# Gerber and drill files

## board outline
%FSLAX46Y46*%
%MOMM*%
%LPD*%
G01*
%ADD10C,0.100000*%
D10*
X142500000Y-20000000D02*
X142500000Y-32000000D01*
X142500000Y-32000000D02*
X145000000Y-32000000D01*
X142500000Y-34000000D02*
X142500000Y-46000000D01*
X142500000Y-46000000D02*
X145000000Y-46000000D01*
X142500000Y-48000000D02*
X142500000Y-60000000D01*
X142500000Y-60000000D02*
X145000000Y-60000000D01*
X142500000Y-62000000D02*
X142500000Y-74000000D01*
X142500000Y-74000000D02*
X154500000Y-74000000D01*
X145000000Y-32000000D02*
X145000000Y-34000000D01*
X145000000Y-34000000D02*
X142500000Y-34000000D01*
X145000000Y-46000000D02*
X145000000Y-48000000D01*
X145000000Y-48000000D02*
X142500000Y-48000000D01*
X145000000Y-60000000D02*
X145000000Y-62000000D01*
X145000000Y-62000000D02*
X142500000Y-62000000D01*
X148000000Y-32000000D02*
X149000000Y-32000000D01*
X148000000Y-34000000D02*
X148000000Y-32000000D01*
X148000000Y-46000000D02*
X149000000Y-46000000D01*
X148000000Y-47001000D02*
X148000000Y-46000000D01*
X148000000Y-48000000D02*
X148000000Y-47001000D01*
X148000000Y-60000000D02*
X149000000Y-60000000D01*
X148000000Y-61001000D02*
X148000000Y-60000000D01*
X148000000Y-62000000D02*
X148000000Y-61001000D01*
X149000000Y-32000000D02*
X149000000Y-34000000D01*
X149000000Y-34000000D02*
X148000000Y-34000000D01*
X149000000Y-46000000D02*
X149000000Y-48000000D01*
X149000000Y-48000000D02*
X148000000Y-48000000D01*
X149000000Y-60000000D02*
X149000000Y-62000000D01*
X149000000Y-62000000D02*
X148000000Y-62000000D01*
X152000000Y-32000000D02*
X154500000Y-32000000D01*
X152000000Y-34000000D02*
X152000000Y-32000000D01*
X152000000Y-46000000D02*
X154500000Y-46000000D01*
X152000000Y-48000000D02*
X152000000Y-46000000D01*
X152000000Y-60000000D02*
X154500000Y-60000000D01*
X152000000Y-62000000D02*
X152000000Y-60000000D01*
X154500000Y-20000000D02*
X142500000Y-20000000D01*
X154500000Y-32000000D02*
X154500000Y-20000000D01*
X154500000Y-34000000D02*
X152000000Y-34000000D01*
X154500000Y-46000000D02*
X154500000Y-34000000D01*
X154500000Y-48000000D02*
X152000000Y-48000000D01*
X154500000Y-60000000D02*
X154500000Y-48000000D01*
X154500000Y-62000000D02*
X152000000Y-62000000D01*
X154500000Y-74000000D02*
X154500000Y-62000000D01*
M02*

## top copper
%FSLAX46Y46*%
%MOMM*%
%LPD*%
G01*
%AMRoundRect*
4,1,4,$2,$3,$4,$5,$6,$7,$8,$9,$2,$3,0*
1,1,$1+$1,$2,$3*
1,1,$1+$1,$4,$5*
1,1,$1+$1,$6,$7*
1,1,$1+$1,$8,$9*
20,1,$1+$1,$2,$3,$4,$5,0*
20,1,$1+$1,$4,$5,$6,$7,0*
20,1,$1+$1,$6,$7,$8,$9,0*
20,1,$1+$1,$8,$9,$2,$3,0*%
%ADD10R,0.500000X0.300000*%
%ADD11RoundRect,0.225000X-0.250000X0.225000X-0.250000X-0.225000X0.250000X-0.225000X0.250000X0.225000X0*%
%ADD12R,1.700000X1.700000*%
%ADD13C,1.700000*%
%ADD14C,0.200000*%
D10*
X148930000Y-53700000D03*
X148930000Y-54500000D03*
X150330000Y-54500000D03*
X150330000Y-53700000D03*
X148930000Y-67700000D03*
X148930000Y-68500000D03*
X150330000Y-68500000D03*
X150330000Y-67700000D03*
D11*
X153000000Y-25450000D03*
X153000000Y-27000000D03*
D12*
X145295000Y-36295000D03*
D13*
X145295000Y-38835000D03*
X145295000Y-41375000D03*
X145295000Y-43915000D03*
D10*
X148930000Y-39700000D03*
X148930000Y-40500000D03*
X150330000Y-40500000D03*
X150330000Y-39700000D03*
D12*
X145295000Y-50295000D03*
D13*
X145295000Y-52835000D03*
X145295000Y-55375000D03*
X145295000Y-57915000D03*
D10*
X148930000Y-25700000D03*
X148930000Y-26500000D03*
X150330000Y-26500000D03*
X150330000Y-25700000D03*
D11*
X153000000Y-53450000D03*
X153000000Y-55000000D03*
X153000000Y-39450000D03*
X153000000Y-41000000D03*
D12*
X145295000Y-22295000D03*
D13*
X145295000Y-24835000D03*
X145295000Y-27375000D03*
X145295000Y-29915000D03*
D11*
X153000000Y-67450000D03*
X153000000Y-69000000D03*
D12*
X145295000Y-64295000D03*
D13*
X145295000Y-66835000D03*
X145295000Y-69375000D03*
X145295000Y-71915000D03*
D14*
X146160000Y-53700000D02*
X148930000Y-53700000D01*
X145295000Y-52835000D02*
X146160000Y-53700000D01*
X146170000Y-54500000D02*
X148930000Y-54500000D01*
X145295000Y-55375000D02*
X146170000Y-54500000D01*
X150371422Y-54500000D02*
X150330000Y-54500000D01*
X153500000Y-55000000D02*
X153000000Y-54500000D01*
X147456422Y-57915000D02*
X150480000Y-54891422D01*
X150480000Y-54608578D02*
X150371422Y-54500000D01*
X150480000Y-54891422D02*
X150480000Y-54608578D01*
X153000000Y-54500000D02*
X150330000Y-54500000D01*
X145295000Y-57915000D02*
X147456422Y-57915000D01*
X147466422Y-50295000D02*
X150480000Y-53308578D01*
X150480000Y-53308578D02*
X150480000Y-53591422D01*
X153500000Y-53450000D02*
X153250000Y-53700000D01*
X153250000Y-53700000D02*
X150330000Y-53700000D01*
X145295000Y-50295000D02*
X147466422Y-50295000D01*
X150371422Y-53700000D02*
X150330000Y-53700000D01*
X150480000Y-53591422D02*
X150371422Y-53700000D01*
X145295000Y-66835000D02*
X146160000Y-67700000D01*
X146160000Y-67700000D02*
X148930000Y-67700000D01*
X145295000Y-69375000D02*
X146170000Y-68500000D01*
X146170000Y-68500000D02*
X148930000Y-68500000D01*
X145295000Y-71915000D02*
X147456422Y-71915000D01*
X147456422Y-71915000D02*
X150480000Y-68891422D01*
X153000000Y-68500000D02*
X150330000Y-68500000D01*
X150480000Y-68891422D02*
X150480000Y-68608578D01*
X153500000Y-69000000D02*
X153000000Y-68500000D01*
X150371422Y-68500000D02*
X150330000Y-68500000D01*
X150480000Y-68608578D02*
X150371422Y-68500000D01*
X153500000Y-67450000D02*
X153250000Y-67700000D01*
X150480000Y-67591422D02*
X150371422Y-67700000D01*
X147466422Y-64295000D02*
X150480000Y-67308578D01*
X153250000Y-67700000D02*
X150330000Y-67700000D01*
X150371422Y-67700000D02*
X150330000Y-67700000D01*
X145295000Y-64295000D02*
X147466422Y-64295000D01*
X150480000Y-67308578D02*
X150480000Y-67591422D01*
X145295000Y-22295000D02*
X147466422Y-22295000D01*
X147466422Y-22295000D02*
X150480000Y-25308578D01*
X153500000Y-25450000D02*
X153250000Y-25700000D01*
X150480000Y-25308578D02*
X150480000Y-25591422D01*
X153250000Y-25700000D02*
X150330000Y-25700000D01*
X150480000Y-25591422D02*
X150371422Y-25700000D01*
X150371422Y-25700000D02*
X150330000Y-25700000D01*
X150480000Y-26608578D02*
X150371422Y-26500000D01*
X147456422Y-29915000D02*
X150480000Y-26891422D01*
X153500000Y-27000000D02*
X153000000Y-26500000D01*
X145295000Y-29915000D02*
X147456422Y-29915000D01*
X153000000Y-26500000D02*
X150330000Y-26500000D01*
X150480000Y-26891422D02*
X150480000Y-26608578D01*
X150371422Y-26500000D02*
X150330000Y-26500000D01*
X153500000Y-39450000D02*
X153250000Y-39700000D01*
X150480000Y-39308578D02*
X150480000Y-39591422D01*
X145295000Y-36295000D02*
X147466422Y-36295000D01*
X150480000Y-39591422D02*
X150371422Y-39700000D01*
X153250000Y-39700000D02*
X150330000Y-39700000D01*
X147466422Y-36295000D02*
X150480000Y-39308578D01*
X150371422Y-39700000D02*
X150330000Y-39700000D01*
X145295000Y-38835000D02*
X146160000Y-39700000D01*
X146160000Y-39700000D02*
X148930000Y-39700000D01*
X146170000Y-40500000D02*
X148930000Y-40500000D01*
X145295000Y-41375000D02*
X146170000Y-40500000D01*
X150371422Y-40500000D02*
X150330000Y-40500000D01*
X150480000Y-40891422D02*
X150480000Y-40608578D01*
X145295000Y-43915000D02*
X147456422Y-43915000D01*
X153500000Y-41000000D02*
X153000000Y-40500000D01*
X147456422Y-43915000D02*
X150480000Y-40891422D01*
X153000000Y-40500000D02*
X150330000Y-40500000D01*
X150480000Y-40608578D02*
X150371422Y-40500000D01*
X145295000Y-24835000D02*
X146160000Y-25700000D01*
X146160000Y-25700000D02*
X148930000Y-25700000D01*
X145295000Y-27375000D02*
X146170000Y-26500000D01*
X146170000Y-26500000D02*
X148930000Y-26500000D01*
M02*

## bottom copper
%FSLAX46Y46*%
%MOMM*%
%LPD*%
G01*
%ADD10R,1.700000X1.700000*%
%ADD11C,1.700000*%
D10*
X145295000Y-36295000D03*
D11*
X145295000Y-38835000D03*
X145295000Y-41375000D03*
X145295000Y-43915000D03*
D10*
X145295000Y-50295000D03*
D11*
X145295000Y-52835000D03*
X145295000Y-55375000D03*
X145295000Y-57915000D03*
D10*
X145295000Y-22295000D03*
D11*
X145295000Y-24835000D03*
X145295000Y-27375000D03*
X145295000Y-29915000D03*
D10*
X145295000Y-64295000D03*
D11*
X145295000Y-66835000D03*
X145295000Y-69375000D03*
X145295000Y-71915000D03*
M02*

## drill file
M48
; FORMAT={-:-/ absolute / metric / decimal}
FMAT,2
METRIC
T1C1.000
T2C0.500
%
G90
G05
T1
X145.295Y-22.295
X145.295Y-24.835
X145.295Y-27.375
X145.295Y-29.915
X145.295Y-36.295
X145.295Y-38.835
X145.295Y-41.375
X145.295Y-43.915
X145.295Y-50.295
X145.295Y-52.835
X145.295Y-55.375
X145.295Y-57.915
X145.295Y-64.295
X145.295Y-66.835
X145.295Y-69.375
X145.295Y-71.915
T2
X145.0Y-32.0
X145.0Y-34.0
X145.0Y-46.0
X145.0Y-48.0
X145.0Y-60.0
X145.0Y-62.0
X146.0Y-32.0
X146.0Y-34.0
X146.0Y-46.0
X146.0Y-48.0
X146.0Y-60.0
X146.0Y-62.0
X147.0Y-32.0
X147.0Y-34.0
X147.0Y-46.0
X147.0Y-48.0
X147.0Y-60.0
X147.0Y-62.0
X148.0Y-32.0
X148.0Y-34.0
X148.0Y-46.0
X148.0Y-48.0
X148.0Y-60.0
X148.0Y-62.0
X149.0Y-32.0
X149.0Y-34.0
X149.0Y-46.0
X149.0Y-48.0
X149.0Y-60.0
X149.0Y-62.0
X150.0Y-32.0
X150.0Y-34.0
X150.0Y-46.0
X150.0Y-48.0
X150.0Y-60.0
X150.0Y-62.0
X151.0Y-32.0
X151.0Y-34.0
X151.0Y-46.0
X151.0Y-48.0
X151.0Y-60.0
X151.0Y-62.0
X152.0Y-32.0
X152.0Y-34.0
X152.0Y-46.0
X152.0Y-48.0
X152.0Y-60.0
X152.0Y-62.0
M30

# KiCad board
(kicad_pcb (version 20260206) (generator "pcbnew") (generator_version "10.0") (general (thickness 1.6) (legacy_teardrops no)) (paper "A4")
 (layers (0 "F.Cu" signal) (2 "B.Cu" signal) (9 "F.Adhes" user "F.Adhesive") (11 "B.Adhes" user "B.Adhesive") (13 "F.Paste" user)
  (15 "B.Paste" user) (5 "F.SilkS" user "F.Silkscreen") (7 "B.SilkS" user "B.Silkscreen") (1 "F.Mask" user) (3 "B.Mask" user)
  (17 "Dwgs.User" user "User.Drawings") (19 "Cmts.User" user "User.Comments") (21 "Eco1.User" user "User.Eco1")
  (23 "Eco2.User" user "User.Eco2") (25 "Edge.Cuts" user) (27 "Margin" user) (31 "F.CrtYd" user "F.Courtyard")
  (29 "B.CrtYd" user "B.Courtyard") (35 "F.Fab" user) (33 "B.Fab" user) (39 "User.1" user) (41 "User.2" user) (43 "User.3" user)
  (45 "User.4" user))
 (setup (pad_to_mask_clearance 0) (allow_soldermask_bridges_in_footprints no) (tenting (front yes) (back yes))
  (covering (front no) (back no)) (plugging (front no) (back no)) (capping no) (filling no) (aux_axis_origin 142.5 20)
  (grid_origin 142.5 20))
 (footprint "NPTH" (layer "F.Cu") (at 150 48)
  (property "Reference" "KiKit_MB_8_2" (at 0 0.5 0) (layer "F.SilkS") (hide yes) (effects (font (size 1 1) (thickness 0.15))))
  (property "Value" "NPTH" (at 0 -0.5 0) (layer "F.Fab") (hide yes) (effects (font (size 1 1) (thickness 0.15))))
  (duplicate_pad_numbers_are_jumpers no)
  (pad "" np_thru_hole circle (at 0 0) (size 0.5 0.5) (drill 0.5) (layers "*.Cu" "*.Mask")))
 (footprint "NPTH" (layer "F.Cu") (at 152 34)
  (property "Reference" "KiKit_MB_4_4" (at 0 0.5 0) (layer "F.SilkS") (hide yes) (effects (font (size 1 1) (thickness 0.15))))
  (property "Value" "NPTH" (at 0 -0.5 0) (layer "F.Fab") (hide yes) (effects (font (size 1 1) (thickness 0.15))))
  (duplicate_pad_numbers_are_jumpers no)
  (pad "" np_thru_hole circle (at 0 0) (size 0.5 0.5) (drill 0.5) (layers "*.Cu" "*.Mask")))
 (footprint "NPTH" (layer "F.Cu") (at 149 62)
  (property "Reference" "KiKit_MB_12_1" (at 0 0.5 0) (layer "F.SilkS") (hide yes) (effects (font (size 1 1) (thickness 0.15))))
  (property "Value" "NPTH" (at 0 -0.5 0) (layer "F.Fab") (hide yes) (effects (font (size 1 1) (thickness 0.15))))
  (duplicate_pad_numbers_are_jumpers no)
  (pad "" np_thru_hole circle (at 0 0) (size 0.5 0.5) (drill 0.5) (layers "*.Cu" "*.Mask")))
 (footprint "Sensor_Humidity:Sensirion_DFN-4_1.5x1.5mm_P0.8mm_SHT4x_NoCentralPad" (layer "F.Cu") (at 149.63 54.1)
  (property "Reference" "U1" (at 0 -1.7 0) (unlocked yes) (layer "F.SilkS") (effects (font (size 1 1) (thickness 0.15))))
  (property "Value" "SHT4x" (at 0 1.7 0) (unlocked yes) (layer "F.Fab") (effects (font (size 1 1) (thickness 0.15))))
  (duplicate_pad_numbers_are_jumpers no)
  (pad "1" smd rect (at -0.7 -0.4) (size 0.5 0.3) (layers "F.Cu" "F.Mask" "F.Paste") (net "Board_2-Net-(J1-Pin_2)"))
  (pad "2" smd rect (at -0.7 0.4) (size 0.5 0.3) (layers "F.Cu" "F.Mask" "F.Paste") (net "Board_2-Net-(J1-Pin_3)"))
  (pad "3" smd rect (at 0.7 0.4) (size 0.5 0.3) (layers "F.Cu" "F.Mask" "F.Paste") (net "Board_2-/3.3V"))
  (pad "4" smd rect (at 0.7 -0.4) (size 0.5 0.3) (layers "F.Cu" "F.Mask" "F.Paste") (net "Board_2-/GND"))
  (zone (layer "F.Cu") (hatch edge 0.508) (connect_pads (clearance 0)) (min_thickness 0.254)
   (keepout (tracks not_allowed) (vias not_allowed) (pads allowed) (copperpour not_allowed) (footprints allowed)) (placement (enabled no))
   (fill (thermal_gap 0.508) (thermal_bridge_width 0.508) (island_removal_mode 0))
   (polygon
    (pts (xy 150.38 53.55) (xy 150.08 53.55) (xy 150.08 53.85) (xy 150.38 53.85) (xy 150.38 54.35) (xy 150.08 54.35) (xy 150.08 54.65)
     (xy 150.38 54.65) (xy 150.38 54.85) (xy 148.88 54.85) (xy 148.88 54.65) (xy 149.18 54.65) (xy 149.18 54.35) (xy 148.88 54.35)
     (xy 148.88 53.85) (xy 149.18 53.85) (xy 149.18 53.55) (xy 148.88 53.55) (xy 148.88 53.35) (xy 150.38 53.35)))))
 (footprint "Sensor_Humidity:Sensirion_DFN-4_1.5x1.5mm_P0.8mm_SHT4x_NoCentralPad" (layer "F.Cu") (at 149.63 68.1)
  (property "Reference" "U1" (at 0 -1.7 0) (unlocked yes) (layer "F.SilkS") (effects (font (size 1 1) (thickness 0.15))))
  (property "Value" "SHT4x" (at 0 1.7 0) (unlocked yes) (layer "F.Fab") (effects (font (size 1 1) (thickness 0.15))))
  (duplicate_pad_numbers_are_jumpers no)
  (pad "1" smd rect (at -0.7 -0.4) (size 0.5 0.3) (layers "F.Cu" "F.Mask" "F.Paste") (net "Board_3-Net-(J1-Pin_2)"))
  (pad "2" smd rect (at -0.7 0.4) (size 0.5 0.3) (layers "F.Cu" "F.Mask" "F.Paste") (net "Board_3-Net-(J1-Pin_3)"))
  (pad "3" smd rect (at 0.7 0.4) (size 0.5 0.3) (layers "F.Cu" "F.Mask" "F.Paste") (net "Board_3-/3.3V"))
  (pad "4" smd rect (at 0.7 -0.4) (size 0.5 0.3) (layers "F.Cu" "F.Mask" "F.Paste") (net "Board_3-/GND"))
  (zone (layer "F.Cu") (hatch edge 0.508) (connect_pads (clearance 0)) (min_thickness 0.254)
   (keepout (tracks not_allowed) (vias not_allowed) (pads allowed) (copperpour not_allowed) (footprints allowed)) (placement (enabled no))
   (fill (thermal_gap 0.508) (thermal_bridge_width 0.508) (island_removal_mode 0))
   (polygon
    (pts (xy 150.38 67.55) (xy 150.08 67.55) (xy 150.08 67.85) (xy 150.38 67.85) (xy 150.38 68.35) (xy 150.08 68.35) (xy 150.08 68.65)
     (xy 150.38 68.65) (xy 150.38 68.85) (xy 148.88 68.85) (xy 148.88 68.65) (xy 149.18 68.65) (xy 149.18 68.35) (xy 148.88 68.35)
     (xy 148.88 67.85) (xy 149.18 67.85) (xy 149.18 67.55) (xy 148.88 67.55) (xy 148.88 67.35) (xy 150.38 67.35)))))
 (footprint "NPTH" (layer "F.Cu") (at 147 48)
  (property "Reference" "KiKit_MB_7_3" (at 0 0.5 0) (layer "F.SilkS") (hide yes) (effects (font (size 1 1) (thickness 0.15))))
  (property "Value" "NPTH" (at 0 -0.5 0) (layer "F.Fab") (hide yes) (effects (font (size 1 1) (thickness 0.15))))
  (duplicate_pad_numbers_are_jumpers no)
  (pad "" np_thru_hole circle (at 0 0) (size 0.5 0.5) (drill 0.5) (layers "*.Cu" "*.Mask")))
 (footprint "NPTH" (layer "F.Cu") (at 146 46)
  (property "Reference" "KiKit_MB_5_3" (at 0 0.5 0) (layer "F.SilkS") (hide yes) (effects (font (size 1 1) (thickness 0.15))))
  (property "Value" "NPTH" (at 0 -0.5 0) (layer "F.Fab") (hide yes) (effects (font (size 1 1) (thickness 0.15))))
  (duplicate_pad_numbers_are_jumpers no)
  (pad "" np_thru_hole circle (at 0 0) (size 0.5 0.5) (drill 0.5) (layers "*.Cu" "*.Mask")))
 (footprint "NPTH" (layer "F.Cu") (at 145 34)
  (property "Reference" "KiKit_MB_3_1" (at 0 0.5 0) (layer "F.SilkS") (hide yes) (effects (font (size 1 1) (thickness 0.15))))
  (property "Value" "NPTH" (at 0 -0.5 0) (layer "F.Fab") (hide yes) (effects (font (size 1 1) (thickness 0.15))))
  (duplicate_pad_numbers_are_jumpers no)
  (pad "" np_thru_hole circle (at 0 0) (size 0.5 0.5) (drill 0.5) (layers "*.Cu" "*.Mask")))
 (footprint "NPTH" (layer "F.Cu") (at 145 62)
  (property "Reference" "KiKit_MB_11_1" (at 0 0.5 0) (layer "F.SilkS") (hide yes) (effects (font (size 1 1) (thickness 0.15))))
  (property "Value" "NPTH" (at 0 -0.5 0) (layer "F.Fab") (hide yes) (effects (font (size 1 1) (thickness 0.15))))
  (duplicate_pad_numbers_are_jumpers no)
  (pad "" np_thru_hole circle (at 0 0) (size 0.5 0.5) (drill 0.5) (layers "*.Cu" "*.Mask")))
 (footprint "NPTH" (layer "F.Cu") (at 151 62)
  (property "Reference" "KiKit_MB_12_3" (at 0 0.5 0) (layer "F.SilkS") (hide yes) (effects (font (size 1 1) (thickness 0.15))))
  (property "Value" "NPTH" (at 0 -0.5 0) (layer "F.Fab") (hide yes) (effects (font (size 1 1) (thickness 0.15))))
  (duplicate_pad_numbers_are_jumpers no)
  (pad "" np_thru_hole circle (at 0 0) (size 0.5 0.5) (drill 0.5) (layers "*.Cu" "*.Mask")))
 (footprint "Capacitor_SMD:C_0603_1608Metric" (layer "F.Cu") (at 153 26.225 -90)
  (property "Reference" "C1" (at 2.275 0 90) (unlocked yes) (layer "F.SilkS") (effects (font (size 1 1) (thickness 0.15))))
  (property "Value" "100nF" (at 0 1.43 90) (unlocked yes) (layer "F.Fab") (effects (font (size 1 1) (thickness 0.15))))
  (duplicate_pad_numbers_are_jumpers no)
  (pad "1" smd roundrect (at -0.775 0 270) (size 0.9 0.95) (layers "F.Cu" "F.Mask" "F.Paste") (roundrect_rratio 0.25) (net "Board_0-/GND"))
  (pad "2" smd roundrect (at 0.775 0 270) (size 0.9 0.95) (layers "F.Cu" "F.Mask" "F.Paste") (roundrect_rratio 0.25) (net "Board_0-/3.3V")))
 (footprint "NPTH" (layer "F.Cu") (at 149 48)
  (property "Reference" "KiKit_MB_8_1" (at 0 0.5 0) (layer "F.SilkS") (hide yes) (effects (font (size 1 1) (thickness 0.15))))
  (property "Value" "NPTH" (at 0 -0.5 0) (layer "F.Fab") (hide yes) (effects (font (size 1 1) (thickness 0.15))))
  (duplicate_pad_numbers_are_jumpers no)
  (pad "" np_thru_hole circle (at 0 0) (size 0.5 0.5) (drill 0.5) (layers "*.Cu" "*.Mask")))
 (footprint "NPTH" (layer "F.Cu") (at 148 32)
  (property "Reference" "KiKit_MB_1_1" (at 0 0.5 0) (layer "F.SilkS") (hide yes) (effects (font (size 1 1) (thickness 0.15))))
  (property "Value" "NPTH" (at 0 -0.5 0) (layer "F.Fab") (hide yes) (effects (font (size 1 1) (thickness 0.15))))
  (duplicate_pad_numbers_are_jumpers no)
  (pad "" np_thru_hole circle (at 0 0) (size 0.5 0.5) (drill 0.5) (layers "*.Cu" "*.Mask")))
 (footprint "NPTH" (layer "F.Cu") (at 145 32)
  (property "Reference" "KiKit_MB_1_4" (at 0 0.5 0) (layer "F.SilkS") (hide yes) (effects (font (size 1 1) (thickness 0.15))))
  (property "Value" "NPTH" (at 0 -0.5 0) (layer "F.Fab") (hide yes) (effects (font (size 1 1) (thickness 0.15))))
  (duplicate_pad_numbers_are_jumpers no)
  (pad "" np_thru_hole circle (at 0 0) (size 0.5 0.5) (drill 0.5) (layers "*.Cu" "*.Mask")))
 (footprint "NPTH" (layer "F.Cu") (at 147 32)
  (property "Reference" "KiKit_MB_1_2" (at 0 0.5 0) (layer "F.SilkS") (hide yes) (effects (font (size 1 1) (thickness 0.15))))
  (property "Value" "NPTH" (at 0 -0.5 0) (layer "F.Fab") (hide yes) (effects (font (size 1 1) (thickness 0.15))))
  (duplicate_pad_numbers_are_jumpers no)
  (pad "" np_thru_hole circle (at 0 0) (size 0.5 0.5) (drill 0.5) (layers "*.Cu" "*.Mask")))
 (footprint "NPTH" (layer "F.Cu") (at 146 48)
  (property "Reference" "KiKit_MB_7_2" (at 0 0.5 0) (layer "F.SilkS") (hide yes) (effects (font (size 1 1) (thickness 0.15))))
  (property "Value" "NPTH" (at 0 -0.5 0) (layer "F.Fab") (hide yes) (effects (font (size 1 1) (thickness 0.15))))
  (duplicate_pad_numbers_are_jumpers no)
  (pad "" np_thru_hole circle (at 0 0) (size 0.5 0.5) (drill 0.5) (layers "*.Cu" "*.Mask")))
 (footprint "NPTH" (layer "F.Cu") (at 146 60)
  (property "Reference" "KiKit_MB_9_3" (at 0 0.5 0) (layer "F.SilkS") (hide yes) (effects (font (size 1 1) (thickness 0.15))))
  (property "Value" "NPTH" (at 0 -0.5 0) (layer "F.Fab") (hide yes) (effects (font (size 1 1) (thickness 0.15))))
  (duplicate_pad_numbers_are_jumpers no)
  (pad "" np_thru_hole circle (at 0 0) (size 0.5 0.5) (drill 0.5) (layers "*.Cu" "*.Mask")))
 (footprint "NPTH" (layer "F.Cu") (at 152 62)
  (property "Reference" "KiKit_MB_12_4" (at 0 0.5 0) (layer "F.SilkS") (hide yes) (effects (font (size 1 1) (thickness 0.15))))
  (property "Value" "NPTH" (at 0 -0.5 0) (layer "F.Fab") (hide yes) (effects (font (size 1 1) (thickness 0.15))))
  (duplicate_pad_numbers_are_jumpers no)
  (pad "" np_thru_hole circle (at 0 0) (size 0.5 0.5) (drill 0.5) (layers "*.Cu" "*.Mask")))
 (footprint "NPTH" (layer "F.Cu") (at 148 60)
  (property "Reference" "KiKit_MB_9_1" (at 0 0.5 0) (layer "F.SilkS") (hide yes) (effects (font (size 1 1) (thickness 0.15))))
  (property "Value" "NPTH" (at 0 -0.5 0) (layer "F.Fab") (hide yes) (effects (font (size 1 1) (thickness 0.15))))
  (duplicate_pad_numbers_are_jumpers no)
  (pad "" np_thru_hole circle (at 0 0) (size 0.5 0.5) (drill 0.5) (layers "*.Cu" "*.Mask")))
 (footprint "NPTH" (layer "F.Cu") (at 150 62)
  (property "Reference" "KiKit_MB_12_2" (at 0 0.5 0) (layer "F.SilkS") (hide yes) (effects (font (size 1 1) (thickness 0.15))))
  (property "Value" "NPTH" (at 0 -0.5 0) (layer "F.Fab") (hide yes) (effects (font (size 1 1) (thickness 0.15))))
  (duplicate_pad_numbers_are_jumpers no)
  (pad "" np_thru_hole circle (at 0 0) (size 0.5 0.5) (drill 0.5) (layers "*.Cu" "*.Mask")))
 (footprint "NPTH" (layer "F.Cu") (at 150 46)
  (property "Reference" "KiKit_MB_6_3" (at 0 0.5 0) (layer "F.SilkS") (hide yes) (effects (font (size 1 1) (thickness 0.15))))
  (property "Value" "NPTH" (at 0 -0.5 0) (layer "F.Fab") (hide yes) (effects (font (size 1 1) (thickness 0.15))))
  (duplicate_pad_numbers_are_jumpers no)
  (pad "" np_thru_hole circle (at 0 0) (size 0.5 0.5) (drill 0.5) (layers "*.Cu" "*.Mask")))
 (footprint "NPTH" (layer "F.Cu") (at 147 60)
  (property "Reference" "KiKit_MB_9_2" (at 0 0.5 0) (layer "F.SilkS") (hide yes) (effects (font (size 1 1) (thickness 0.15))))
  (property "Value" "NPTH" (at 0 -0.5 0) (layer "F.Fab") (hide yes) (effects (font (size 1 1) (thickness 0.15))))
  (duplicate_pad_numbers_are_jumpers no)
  (pad "" np_thru_hole circle (at 0 0) (size 0.5 0.5) (drill 0.5) (layers "*.Cu" "*.Mask")))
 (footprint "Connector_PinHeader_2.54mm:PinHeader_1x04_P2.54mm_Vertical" (layer "F.Cu") (at 145.295 36.295)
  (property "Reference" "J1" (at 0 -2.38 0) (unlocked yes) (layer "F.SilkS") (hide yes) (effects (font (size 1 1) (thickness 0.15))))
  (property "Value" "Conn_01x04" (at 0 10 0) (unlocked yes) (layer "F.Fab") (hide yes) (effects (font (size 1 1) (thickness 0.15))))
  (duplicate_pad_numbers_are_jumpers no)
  (pad "1" thru_hole rect (at 0 0) (size 1.7 1.7) (drill 1) (layers "*.Cu" "*.Mask") (remove_unused_layers no) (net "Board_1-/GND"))
  (pad "2" thru_hole circle (at 0 2.54) (size 1.7 1.7) (drill 1) (layers "*.Cu" "*.Mask") (remove_unused_layers no)
   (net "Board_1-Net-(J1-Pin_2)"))
  (pad "3" thru_hole circle (at 0 5.08) (size 1.7 1.7) (drill 1) (layers "*.Cu" "*.Mask") (remove_unused_layers no)
   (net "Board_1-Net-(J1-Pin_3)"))
  (pad "4" thru_hole circle (at 0 7.62) (size 1.7 1.7) (drill 1) (layers "*.Cu" "*.Mask") (remove_unused_layers no) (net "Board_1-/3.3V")))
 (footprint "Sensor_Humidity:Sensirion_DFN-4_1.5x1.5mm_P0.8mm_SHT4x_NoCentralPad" (layer "F.Cu") (at 149.63 40.1)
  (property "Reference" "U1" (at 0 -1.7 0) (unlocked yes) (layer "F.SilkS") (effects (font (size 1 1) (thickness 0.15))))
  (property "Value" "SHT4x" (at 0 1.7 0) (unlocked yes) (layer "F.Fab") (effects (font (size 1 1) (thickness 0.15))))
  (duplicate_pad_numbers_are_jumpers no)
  (pad "1" smd rect (at -0.7 -0.4) (size 0.5 0.3) (layers "F.Cu" "F.Mask" "F.Paste") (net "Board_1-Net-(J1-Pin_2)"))
  (pad "2" smd rect (at -0.7 0.4) (size 0.5 0.3) (layers "F.Cu" "F.Mask" "F.Paste") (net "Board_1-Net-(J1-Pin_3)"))
  (pad "3" smd rect (at 0.7 0.4) (size 0.5 0.3) (layers "F.Cu" "F.Mask" "F.Paste") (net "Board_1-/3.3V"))
  (pad "4" smd rect (at 0.7 -0.4) (size 0.5 0.3) (layers "F.Cu" "F.Mask" "F.Paste") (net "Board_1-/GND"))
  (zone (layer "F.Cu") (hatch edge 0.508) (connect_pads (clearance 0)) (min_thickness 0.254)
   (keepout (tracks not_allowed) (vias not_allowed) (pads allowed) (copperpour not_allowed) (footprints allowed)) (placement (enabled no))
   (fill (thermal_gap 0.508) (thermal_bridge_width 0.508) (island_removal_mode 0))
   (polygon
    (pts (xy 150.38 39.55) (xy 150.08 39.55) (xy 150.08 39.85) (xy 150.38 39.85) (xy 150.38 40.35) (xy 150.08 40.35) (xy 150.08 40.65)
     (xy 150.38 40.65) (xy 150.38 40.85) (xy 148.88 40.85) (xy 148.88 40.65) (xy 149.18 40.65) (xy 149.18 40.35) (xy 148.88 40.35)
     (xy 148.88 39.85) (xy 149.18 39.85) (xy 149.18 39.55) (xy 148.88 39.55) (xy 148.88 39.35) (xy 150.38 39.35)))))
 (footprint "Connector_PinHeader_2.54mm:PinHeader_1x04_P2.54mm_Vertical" (layer "F.Cu") (at 145.295 50.295)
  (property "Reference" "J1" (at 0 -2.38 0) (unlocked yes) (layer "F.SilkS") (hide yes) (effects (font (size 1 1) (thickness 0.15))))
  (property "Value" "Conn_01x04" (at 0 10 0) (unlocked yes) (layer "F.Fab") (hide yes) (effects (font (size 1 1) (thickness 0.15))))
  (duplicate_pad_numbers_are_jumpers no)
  (pad "1" thru_hole rect (at 0 0) (size 1.7 1.7) (drill 1) (layers "*.Cu" "*.Mask") (remove_unused_layers no) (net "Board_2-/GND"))
  (pad "2" thru_hole circle (at 0 2.54) (size 1.7 1.7) (drill 1) (layers "*.Cu" "*.Mask") (remove_unused_layers no)
   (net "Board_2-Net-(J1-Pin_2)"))
  (pad "3" thru_hole circle (at 0 5.08) (size 1.7 1.7) (drill 1) (layers "*.Cu" "*.Mask") (remove_unused_layers no)
   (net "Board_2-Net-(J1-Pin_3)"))
  (pad "4" thru_hole circle (at 0 7.62) (size 1.7 1.7) (drill 1) (layers "*.Cu" "*.Mask") (remove_unused_layers no) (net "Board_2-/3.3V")))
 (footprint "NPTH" (layer "F.Cu") (at 151 32)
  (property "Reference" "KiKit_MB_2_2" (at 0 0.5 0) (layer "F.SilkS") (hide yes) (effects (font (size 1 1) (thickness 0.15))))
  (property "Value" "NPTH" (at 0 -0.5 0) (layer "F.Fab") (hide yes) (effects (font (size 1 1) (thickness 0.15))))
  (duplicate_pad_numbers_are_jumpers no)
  (pad "" np_thru_hole circle (at 0 0) (size 0.5 0.5) (drill 0.5) (layers "*.Cu" "*.Mask")))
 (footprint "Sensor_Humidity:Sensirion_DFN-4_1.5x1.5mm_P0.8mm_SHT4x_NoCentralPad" (layer "F.Cu") (at 149.63 26.1)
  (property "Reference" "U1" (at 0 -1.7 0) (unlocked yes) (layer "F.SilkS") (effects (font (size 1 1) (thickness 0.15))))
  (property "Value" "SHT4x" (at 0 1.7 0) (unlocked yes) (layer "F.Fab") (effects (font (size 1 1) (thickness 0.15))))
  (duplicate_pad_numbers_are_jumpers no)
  (pad "1" smd rect (at -0.7 -0.4) (size 0.5 0.3) (layers "F.Cu" "F.Mask" "F.Paste") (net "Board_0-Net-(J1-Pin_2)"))
  (pad "2" smd rect (at -0.7 0.4) (size 0.5 0.3) (layers "F.Cu" "F.Mask" "F.Paste") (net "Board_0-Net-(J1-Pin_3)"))
  (pad "3" smd rect (at 0.7 0.4) (size 0.5 0.3) (layers "F.Cu" "F.Mask" "F.Paste") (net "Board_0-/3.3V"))
  (pad "4" smd rect (at 0.7 -0.4) (size 0.5 0.3) (layers "F.Cu" "F.Mask" "F.Paste") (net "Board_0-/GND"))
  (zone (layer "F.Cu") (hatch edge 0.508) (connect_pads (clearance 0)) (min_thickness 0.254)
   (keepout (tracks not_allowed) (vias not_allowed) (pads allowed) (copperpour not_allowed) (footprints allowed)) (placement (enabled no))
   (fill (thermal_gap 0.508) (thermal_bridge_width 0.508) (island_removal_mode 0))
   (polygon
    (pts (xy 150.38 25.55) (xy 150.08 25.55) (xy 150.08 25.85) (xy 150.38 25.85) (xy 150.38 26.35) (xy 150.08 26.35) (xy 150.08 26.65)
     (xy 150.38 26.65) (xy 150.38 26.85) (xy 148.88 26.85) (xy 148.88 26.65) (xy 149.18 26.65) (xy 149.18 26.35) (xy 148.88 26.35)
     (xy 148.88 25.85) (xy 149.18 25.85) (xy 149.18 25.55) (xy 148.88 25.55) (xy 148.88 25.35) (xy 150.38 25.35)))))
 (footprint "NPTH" (layer "F.Cu") (at 152 60)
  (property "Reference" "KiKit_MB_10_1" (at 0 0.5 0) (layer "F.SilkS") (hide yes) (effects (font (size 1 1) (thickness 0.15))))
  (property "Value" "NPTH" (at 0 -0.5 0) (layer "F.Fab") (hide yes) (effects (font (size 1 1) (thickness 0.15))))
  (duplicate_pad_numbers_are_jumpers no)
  (pad "" np_thru_hole circle (at 0 0) (size 0.5 0.5) (drill 0.5) (layers "*.Cu" "*.Mask")))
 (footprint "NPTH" (layer "F.Cu") (at 148 34)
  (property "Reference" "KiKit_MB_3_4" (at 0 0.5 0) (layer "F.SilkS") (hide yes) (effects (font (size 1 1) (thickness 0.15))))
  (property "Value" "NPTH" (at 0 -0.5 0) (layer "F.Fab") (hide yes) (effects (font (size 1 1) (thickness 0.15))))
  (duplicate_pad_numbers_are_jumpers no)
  (pad "" np_thru_hole circle (at 0 0) (size 0.5 0.5) (drill 0.5) (layers "*.Cu" "*.Mask")))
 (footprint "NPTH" (layer "F.Cu") (at 145 48)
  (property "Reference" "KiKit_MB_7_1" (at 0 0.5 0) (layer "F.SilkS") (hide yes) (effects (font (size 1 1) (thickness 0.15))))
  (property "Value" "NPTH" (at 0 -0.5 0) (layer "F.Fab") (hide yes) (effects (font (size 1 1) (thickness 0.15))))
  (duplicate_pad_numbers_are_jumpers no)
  (pad "" np_thru_hole circle (at 0 0) (size 0.5 0.5) (drill 0.5) (layers "*.Cu" "*.Mask")))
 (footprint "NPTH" (layer "F.Cu") (at 149 32)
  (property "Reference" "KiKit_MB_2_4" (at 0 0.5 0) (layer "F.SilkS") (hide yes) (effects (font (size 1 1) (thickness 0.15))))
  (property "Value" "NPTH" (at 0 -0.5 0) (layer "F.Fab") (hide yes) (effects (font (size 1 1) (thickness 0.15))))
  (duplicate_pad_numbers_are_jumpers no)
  (pad "" np_thru_hole circle (at 0 0) (size 0.5 0.5) (drill 0.5) (layers "*.Cu" "*.Mask")))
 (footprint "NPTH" (layer "F.Cu") (at 148 62)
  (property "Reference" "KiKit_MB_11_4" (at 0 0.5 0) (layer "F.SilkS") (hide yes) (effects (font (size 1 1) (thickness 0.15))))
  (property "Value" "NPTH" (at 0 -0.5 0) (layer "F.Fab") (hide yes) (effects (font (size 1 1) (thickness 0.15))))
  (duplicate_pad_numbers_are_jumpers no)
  (pad "" np_thru_hole circle (at 0 0) (size 0.5 0.5) (drill 0.5) (layers "*.Cu" "*.Mask")))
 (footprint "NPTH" (layer "F.Cu") (at 151 48)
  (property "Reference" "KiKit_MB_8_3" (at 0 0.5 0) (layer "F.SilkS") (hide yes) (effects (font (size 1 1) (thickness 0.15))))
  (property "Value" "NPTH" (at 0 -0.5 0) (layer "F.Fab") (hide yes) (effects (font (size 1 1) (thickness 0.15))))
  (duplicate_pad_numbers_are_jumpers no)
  (pad "" np_thru_hole circle (at 0 0) (size 0.5 0.5) (drill 0.5) (layers "*.Cu" "*.Mask")))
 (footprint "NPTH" (layer "F.Cu") (at 148 48)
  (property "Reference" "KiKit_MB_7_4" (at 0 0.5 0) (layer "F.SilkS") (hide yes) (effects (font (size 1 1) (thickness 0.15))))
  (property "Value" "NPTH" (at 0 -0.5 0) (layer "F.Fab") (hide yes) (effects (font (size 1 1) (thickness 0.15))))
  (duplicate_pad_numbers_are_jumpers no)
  (pad "" np_thru_hole circle (at 0 0) (size 0.5 0.5) (drill 0.5) (layers "*.Cu" "*.Mask")))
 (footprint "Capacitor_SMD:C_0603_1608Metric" (layer "F.Cu") (at 153 54.225 -90)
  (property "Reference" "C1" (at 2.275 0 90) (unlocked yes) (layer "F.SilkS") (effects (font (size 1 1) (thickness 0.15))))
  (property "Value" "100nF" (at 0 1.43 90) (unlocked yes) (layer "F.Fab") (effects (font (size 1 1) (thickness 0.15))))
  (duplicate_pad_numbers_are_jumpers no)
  (pad "1" smd roundrect (at -0.775 0 270) (size 0.9 0.95) (layers "F.Cu" "F.Mask" "F.Paste") (roundrect_rratio 0.25) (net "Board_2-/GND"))
  (pad "2" smd roundrect (at 0.775 0 270) (size 0.9 0.95) (layers "F.Cu" "F.Mask" "F.Paste") (roundrect_rratio 0.25) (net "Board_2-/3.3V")))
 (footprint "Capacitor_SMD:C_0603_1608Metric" (layer "F.Cu") (at 153 40.225 -90)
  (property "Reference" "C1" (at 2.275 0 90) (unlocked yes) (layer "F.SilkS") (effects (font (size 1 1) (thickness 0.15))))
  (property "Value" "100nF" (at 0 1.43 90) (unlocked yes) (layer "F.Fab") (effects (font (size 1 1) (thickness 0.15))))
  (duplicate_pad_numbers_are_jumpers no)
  (pad "1" smd roundrect (at -0.775 0 270) (size 0.9 0.95) (layers "F.Cu" "F.Mask" "F.Paste") (roundrect_rratio 0.25) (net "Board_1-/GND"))
  (pad "2" smd roundrect (at 0.775 0 270) (size 0.9 0.95) (layers "F.Cu" "F.Mask" "F.Paste") (roundrect_rratio 0.25) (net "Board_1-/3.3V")))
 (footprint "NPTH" (layer "F.Cu") (at 152 32)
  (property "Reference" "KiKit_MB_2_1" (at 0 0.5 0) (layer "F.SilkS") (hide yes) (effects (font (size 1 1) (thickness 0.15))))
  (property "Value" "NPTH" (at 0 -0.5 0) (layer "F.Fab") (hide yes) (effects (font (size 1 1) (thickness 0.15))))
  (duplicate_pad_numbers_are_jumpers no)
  (pad "" np_thru_hole circle (at 0 0) (size 0.5 0.5) (drill 0.5) (layers "*.Cu" "*.Mask")))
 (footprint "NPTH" (layer "F.Cu") (at 146 62)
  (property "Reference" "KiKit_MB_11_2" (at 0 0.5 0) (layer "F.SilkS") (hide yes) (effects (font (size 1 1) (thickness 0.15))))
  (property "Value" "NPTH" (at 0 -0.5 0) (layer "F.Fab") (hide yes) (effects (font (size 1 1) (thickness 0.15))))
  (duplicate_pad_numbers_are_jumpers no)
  (pad "" np_thru_hole circle (at 0 0) (size 0.5 0.5) (drill 0.5) (layers "*.Cu" "*.Mask")))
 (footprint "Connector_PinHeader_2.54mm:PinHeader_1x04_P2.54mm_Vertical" (layer "F.Cu") (at 145.295 22.295)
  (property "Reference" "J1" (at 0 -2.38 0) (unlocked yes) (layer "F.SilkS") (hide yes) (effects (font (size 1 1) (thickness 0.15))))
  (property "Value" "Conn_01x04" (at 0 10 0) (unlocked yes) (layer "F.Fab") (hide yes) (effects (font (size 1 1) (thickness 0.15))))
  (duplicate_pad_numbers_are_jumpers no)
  (pad "1" thru_hole rect (at 0 0) (size 1.7 1.7) (drill 1) (layers "*.Cu" "*.Mask") (remove_unused_layers no) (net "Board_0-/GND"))
  (pad "2" thru_hole circle (at 0 2.54) (size 1.7 1.7) (drill 1) (layers "*.Cu" "*.Mask") (remove_unused_layers no)
   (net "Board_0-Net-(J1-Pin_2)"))
  (pad "3" thru_hole circle (at 0 5.08) (size 1.7 1.7) (drill 1) (layers "*.Cu" "*.Mask") (remove_unused_layers no)
   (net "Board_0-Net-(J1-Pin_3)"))
  (pad "4" thru_hole circle (at 0 7.62) (size 1.7 1.7) (drill 1) (layers "*.Cu" "*.Mask") (remove_unused_layers no) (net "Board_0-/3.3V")))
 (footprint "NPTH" (layer "F.Cu") (at 146 34)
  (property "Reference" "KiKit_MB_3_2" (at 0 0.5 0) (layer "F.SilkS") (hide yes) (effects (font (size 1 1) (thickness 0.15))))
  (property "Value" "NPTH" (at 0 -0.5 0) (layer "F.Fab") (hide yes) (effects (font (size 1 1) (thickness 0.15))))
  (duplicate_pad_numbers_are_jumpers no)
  (pad "" np_thru_hole circle (at 0 0) (size 0.5 0.5) (drill 0.5) (layers "*.Cu" "*.Mask")))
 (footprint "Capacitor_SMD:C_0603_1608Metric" (layer "F.Cu") (at 153 68.225 -90)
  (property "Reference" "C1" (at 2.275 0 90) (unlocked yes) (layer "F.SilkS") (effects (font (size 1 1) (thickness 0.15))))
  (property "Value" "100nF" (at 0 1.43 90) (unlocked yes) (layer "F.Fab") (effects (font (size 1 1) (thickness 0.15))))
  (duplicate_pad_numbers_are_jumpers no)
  (pad "1" smd roundrect (at -0.775 0 270) (size 0.9 0.95) (layers "F.Cu" "F.Mask" "F.Paste") (roundrect_rratio 0.25) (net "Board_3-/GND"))
  (pad "2" smd roundrect (at 0.775 0 270) (size 0.9 0.95) (layers "F.Cu" "F.Mask" "F.Paste") (roundrect_rratio 0.25) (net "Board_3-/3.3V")))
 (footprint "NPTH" (layer "F.Cu") (at 146 32)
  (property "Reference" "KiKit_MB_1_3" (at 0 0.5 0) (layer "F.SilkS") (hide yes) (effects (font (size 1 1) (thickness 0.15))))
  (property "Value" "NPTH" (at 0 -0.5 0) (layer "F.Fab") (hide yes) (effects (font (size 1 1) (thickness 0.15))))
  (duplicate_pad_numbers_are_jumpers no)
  (pad "" np_thru_hole circle (at 0 0) (size 0.5 0.5) (drill 0.5) (layers "*.Cu" "*.Mask")))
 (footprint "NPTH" (layer "F.Cu") (at 150 32)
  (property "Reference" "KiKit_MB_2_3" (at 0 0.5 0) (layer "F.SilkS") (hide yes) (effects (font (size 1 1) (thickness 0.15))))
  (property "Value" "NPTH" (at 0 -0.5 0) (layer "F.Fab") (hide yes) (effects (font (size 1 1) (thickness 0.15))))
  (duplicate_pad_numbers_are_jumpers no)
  (pad "" np_thru_hole circle (at 0 0) (size 0.5 0.5) (drill 0.5) (layers "*.Cu" "*.Mask")))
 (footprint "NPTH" (layer "F.Cu") (at 149 34)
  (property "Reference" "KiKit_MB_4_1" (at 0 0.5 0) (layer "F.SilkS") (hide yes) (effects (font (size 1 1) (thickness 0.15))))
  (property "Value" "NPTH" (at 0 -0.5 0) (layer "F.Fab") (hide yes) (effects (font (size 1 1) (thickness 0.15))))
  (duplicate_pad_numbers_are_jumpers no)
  (pad "" np_thru_hole circle (at 0 0) (size 0.5 0.5) (drill 0.5) (layers "*.Cu" "*.Mask")))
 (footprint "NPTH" (layer "F.Cu") (at 150 34)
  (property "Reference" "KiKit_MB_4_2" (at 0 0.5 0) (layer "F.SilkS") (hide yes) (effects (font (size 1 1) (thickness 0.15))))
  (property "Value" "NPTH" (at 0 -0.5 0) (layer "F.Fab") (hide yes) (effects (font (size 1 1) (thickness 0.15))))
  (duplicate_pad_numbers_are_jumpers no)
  (pad "" np_thru_hole circle (at 0 0) (size 0.5 0.5) (drill 0.5) (layers "*.Cu" "*.Mask")))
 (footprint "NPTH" (layer "F.Cu") (at 145 60)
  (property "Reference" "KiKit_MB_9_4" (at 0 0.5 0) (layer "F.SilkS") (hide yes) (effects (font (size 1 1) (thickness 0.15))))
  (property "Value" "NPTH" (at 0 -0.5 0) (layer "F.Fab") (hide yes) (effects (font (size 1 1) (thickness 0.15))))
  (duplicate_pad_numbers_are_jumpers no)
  (pad "" np_thru_hole circle (at 0 0) (size 0.5 0.5) (drill 0.5) (layers "*.Cu" "*.Mask")))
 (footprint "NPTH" (layer "F.Cu") (at 151 34)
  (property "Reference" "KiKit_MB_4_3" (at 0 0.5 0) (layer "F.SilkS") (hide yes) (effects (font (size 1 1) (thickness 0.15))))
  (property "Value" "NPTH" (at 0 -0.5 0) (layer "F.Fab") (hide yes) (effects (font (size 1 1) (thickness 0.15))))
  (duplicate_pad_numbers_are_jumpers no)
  (pad "" np_thru_hole circle (at 0 0) (size 0.5 0.5) (drill 0.5) (layers "*.Cu" "*.Mask")))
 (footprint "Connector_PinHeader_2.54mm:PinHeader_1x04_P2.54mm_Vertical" (layer "F.Cu") (at 145.295 64.295)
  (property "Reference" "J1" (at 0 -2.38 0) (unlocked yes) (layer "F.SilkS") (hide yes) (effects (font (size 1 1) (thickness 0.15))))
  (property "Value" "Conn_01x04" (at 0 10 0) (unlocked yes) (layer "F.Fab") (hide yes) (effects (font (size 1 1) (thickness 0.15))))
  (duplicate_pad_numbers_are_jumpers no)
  (pad "1" thru_hole rect (at 0 0) (size 1.7 1.7) (drill 1) (layers "*.Cu" "*.Mask") (remove_unused_layers no) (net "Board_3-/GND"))
  (pad "2" thru_hole circle (at 0 2.54) (size 1.7 1.7) (drill 1) (layers "*.Cu" "*.Mask") (remove_unused_layers no)
   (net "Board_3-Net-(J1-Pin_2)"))
  (pad "3" thru_hole circle (at 0 5.08) (size 1.7 1.7) (drill 1) (layers "*.Cu" "*.Mask") (remove_unused_layers no)
   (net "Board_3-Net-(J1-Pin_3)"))
  (pad "4" thru_hole circle (at 0 7.62) (size 1.7 1.7) (drill 1) (layers "*.Cu" "*.Mask") (remove_unused_layers no) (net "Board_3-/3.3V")))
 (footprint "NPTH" (layer "F.Cu") (at 150 60)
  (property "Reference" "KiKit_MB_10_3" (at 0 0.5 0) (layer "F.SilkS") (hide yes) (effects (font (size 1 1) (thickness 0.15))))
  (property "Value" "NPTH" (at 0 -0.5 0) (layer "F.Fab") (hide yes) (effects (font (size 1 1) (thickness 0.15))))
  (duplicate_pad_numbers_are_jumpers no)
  (pad "" np_thru_hole circle (at 0 0) (size 0.5 0.5) (drill 0.5) (layers "*.Cu" "*.Mask")))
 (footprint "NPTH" (layer "F.Cu") (at 149 46)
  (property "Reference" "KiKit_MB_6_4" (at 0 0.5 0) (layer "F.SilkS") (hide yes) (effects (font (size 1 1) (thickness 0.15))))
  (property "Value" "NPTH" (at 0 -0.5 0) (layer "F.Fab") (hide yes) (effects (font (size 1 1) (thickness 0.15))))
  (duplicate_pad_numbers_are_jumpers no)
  (pad "" np_thru_hole circle (at 0 0) (size 0.5 0.5) (drill 0.5) (layers "*.Cu" "*.Mask")))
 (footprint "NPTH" (layer "F.Cu") (at 151 46)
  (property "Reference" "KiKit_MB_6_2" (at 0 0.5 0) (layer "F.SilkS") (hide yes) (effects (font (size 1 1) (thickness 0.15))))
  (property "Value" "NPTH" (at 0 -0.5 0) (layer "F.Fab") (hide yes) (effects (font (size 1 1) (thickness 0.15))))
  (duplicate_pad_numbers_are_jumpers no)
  (pad "" np_thru_hole circle (at 0 0) (size 0.5 0.5) (drill 0.5) (layers "*.Cu" "*.Mask")))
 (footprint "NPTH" (layer "F.Cu") (at 152 46)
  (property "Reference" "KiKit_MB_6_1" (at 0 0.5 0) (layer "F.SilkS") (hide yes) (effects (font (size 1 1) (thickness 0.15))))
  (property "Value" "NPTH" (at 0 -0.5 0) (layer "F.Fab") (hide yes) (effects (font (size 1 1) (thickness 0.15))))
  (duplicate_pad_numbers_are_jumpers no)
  (pad "" np_thru_hole circle (at 0 0) (size 0.5 0.5) (drill 0.5) (layers "*.Cu" "*.Mask")))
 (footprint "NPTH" (layer "F.Cu") (at 149 60)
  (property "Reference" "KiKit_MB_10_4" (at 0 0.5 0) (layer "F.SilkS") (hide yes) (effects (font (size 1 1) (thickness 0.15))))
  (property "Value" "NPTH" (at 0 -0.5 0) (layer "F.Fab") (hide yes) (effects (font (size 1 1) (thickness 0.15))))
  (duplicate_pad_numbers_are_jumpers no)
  (pad "" np_thru_hole circle (at 0 0) (size 0.5 0.5) (drill 0.5) (layers "*.Cu" "*.Mask")))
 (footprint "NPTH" (layer "F.Cu") (at 151 60)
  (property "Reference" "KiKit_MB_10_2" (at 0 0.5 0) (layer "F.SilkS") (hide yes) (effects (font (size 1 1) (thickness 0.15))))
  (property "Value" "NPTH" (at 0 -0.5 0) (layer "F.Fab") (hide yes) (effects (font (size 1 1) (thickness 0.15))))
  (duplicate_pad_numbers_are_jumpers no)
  (pad "" np_thru_hole circle (at 0 0) (size 0.5 0.5) (drill 0.5) (layers "*.Cu" "*.Mask")))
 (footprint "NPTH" (layer "F.Cu") (at 152 48)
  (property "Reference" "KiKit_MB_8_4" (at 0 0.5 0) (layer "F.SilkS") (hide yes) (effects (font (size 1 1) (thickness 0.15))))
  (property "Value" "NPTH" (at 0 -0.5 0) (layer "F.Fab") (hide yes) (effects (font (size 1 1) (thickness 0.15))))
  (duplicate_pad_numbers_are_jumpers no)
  (pad "" np_thru_hole circle (at 0 0) (size 0.5 0.5) (drill 0.5) (layers "*.Cu" "*.Mask")))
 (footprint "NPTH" (layer "F.Cu") (at 147 46)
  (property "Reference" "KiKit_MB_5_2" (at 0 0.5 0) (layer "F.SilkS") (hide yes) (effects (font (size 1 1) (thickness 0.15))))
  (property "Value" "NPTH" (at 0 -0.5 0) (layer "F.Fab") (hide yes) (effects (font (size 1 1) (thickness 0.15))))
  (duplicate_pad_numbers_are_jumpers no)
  (pad "" np_thru_hole circle (at 0 0) (size 0.5 0.5) (drill 0.5) (layers "*.Cu" "*.Mask")))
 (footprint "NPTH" (layer "F.Cu") (at 145 46)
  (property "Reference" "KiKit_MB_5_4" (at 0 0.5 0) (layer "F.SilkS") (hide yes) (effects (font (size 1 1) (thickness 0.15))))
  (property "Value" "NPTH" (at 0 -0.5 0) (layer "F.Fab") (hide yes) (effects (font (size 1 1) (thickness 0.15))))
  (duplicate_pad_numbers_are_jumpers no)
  (pad "" np_thru_hole circle (at 0 0) (size 0.5 0.5) (drill 0.5) (layers "*.Cu" "*.Mask")))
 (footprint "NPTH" (layer "F.Cu") (at 147 34)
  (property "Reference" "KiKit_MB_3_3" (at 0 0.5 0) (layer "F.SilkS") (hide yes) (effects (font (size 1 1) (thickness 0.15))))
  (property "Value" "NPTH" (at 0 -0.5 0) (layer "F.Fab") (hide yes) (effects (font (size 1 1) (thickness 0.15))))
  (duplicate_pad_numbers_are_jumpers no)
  (pad "" np_thru_hole circle (at 0 0) (size 0.5 0.5) (drill 0.5) (layers "*.Cu" "*.Mask")))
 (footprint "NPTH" (layer "F.Cu") (at 147 62)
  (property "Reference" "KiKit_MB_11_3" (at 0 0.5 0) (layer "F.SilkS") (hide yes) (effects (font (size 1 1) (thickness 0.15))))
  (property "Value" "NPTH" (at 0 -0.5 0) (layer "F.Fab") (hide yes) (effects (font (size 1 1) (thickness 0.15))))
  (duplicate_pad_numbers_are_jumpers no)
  (pad "" np_thru_hole circle (at 0 0) (size 0.5 0.5) (drill 0.5) (layers "*.Cu" "*.Mask")))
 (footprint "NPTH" (layer "F.Cu") (at 148 46)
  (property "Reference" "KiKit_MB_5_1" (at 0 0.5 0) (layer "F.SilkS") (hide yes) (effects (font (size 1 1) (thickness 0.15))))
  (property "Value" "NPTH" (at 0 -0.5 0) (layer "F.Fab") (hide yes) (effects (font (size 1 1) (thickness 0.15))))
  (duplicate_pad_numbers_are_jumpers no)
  (pad "" np_thru_hole circle (at 0 0) (size 0.5 0.5) (drill 0.5) (layers "*.Cu" "*.Mask")))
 (gr_line (start 142.5 20) (end 142.5 32) (stroke (width 0.1) (type default)) (layer "Edge.Cuts"))
 (gr_line (start 142.5 32) (end 145 32) (stroke (width 0.1) (type default)) (layer "Edge.Cuts"))
 (gr_line (start 142.5 34) (end 142.5 46) (stroke (width 0.1) (type default)) (layer "Edge.Cuts"))
 (gr_line (start 142.5 46) (end 145 46) (stroke (width 0.1) (type default)) (layer "Edge.Cuts"))
 (gr_line (start 142.5 48) (end 142.5 60) (stroke (width 0.1) (type default)) (layer "Edge.Cuts"))
 (gr_line (start 142.5 60) (end 145 60) (stroke (width 0.1) (type default)) (layer "Edge.Cuts"))
 (gr_line (start 142.5 62) (end 142.5 74) (stroke (width 0.1) (type default)) (layer "Edge.Cuts"))
 (gr_line (start 142.5 74) (end 154.5 74) (stroke (width 0.1) (type default)) (layer "Edge.Cuts"))
 (gr_line (start 145 32) (end 145 34) (stroke (width 0.1) (type default)) (layer "Edge.Cuts"))
 (gr_line (start 145 34) (end 142.5 34) (stroke (width 0.1) (type default)) (layer "Edge.Cuts"))
 (gr_line (start 145 46) (end 145 48) (stroke (width 0.1) (type default)) (layer "Edge.Cuts"))
 (gr_line (start 145 48) (end 142.5 48) (stroke (width 0.1) (type default)) (layer "Edge.Cuts"))
 (gr_line (start 145 60) (end 145 62) (stroke (width 0.1) (type default)) (layer "Edge.Cuts"))
 (gr_line (start 145 62) (end 142.5 62) (stroke (width 0.1) (type default)) (layer "Edge.Cuts"))
 (gr_line (start 148 32) (end 149 32) (stroke (width 0.1) (type default)) (layer "Edge.Cuts"))
 (gr_line (start 148 34) (end 148 32) (stroke (width 0.1) (type default)) (layer "Edge.Cuts"))
 (gr_line (start 148 46) (end 149 46) (stroke (width 0.1) (type default)) (layer "Edge.Cuts"))
 (gr_line (start 148 47.001) (end 148 46) (stroke (width 0.1) (type default)) (layer "Edge.Cuts"))
 (gr_line (start 148 48) (end 148 47.001) (stroke (width 0.1) (type default)) (layer "Edge.Cuts"))
 (gr_line (start 148 60) (end 149 60) (stroke (width 0.1) (type default)) (layer "Edge.Cuts"))
 (gr_line (start 148 61.001) (end 148 60) (stroke (width 0.1) (type default)) (layer "Edge.Cuts"))
 (gr_line (start 148 62) (end 148 61.001) (stroke (width 0.1) (type default)) (layer "Edge.Cuts"))
 (gr_line (start 149 32) (end 149 34) (stroke (width 0.1) (type default)) (layer "Edge.Cuts"))
 (gr_line (start 149 34) (end 148 34) (stroke (width 0.1) (type default)) (layer "Edge.Cuts"))
 (gr_line (start 149 46) (end 149 48) (stroke (width 0.1) (type default)) (layer "Edge.Cuts"))
 (gr_line (start 149 48) (end 148 48) (stroke (width 0.1) (type default)) (layer "Edge.Cuts"))
 (gr_line (start 149 60) (end 149 62) (stroke (width 0.1) (type default)) (layer "Edge.Cuts"))
 (gr_line (start 149 62) (end 148 62) (stroke (width 0.1) (type default)) (layer "Edge.Cuts"))
 (gr_line (start 152 32) (end 154.5 32) (stroke (width 0.1) (type default)) (layer "Edge.Cuts"))
 (gr_line (start 152 34) (end 152 32) (stroke (width 0.1) (type default)) (layer "Edge.Cuts"))
 (gr_line (start 152 46) (end 154.5 46) (stroke (width 0.1) (type default)) (layer "Edge.Cuts"))
 (gr_line (start 152 48) (end 152 46) (stroke (width 0.1) (type default)) (layer "Edge.Cuts"))
 (gr_line (start 152 60) (end 154.5 60) (stroke (width 0.1) (type default)) (layer "Edge.Cuts"))
 (gr_line (start 152 62) (end 152 60) (stroke (width 0.1) (type default)) (layer "Edge.Cuts"))
 (gr_line (start 154.5 20) (end 142.5 20) (stroke (width 0.1) (type default)) (layer "Edge.Cuts"))
 (gr_line (start 154.5 32) (end 154.5 20) (stroke (width 0.1) (type default)) (layer "Edge.Cuts"))
 (gr_line (start 154.5 34) (end 152 34) (stroke (width 0.1) (type default)) (layer "Edge.Cuts"))
 (gr_line (start 154.5 46) (end 154.5 34) (stroke (width 0.1) (type default)) (layer "Edge.Cuts"))
 (gr_line (start 154.5 48) (end 152 48) (stroke (width 0.1) (type default)) (layer "Edge.Cuts"))
 (gr_line (start 154.5 60) (end 154.5 48) (stroke (width 0.1) (type default)) (layer "Edge.Cuts"))
 (gr_line (start 154.5 62) (end 152 62) (stroke (width 0.1) (type default)) (layer "Edge.Cuts"))
 (gr_line (start 154.5 74) (end 154.5 62) (stroke (width 0.1) (type default)) (layer "Edge.Cuts"))
 (segment (start 146.16 53.7) (end 148.93 53.7) (width 0.2) (layer "F.Cu") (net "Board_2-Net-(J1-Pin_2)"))
 (segment (start 145.295 52.835) (end 146.16 53.7) (width 0.2) (layer "F.Cu") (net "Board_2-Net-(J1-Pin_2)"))
 (segment (start 146.17 54.5) (end 148.93 54.5) (width 0.2) (layer "F.Cu") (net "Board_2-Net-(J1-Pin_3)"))
 (segment (start 145.295 55.375) (end 146.17 54.5) (width 0.2) (layer "F.Cu") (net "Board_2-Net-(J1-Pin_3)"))
 (segment (start 150.371422 54.5) (end 150.33 54.5) (width 0.2) (layer "F.Cu") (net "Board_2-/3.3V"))
 (segment (start 153.5 55) (end 153 54.5) (width 0.2) (layer "F.Cu") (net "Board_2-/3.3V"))
 (segment (start 147.456422 57.915) (end 150.48 54.891422) (width 0.2) (layer "F.Cu") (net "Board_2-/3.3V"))
 (segment (start 150.48 54.608578) (end 150.371422 54.5) (width 0.2) (layer "F.Cu") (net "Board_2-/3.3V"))
 (segment (start 150.48 54.891422) (end 150.48 54.608578) (width 0.2) (layer "F.Cu") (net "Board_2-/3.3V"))
 (segment (start 153 54.5) (end 150.33 54.5) (width 0.2) (layer "F.Cu") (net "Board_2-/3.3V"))
 (segment (start 145.295 57.915) (end 147.456422 57.915) (width 0.2) (layer "F.Cu") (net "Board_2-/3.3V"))
 (segment (start 147.466422 50.295) (end 150.48 53.308578) (width 0.2) (layer "F.Cu") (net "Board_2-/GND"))
 (segment (start 150.48 53.308578) (end 150.48 53.591422) (width 0.2) (layer "F.Cu") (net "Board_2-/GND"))
 (segment (start 153.5 53.45) (end 153.25 53.7) (width 0.2) (layer "F.Cu") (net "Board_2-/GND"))
 (segment (start 153.25 53.7) (end 150.33 53.7) (width 0.2) (layer "F.Cu") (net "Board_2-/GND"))
 (segment (start 145.295 50.295) (end 147.466422 50.295) (width 0.2) (layer "F.Cu") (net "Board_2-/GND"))
 (segment (start 150.371422 53.7) (end 150.33 53.7) (width 0.2) (layer "F.Cu") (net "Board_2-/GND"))
 (segment (start 150.48 53.591422) (end 150.371422 53.7) (width 0.2) (layer "F.Cu") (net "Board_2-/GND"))
 (segment (start 145.295 66.835) (end 146.16 67.7) (width 0.2) (layer "F.Cu") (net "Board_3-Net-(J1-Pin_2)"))
 (segment (start 146.16 67.7) (end 148.93 67.7) (width 0.2) (layer "F.Cu") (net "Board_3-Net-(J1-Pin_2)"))
 (segment (start 145.295 69.375) (end 146.17 68.5) (width 0.2) (layer "F.Cu") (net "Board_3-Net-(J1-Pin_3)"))
 (segment (start 146.17 68.5) (end 148.93 68.5) (width 0.2) (layer "F.Cu") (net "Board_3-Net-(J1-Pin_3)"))
 (segment (start 145.295 71.915) (end 147.456422 71.915) (width 0.2) (layer "F.Cu") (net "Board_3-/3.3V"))
 (segment (start 147.456422 71.915) (end 150.48 68.891422) (width 0.2) (layer "F.Cu") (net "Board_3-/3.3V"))
 (segment (start 153 68.5) (end 150.33 68.5) (width 0.2) (layer "F.Cu") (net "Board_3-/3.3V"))
 (segment (start 150.48 68.891422) (end 150.48 68.608578) (width 0.2) (layer "F.Cu") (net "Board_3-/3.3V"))
 (segment (start 153.5 69) (end 153 68.5) (width 0.2) (layer "F.Cu") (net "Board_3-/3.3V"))
 (segment (start 150.371422 68.5) (end 150.33 68.5) (width 0.2) (layer "F.Cu") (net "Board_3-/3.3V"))
 (segment (start 150.48 68.608578) (end 150.371422 68.5) (width 0.2) (layer "F.Cu") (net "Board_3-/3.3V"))
 (segment (start 153.5 67.45) (end 153.25 67.7) (width 0.2) (layer "F.Cu") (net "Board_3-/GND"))
 (segment (start 150.48 67.591422) (end 150.371422 67.7) (width 0.2) (layer "F.Cu") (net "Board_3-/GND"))
 (segment (start 147.466422 64.295) (end 150.48 67.308578) (width 0.2) (layer "F.Cu") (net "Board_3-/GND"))
 (segment (start 153.25 67.7) (end 150.33 67.7) (width 0.2) (layer "F.Cu") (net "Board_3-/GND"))
 (segment (start 150.371422 67.7) (end 150.33 67.7) (width 0.2) (layer "F.Cu") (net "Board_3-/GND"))
 (segment (start 145.295 64.295) (end 147.466422 64.295) (width 0.2) (layer "F.Cu") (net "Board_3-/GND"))
 (segment (start 150.48 67.308578) (end 150.48 67.591422) (width 0.2) (layer "F.Cu") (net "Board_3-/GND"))
 (segment (start 145.295 22.295) (end 147.466422 22.295) (width 0.2) (layer "F.Cu") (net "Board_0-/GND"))
 (segment (start 147.466422 22.295) (end 150.48 25.308578) (width 0.2) (layer "F.Cu") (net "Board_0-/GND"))
 (segment (start 153.5 25.45) (end 153.25 25.7) (width 0.2) (layer "F.Cu") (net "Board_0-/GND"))
 (segment (start 150.48 25.308578) (end 150.48 25.591422) (width 0.2) (layer "F.Cu") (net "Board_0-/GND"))
 (segment (start 153.25 25.7) (end 150.33 25.7) (width 0.2) (layer "F.Cu") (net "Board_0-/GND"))
 (segment (start 150.48 25.591422) (end 150.371422 25.7) (width 0.2) (layer "F.Cu") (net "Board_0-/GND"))
 (segment (start 150.371422 25.7) (end 150.33 25.7) (width 0.2) (layer "F.Cu") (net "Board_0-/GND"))
 (segment (start 150.48 26.608578) (end 150.371422 26.5) (width 0.2) (layer "F.Cu") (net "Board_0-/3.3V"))
 (segment (start 147.456422 29.915) (end 150.48 26.891422) (width 0.2) (layer "F.Cu") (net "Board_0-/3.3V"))
 (segment (start 153.5 27) (end 153 26.5) (width 0.2) (layer "F.Cu") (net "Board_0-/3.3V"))
 (segment (start 145.295 29.915) (end 147.456422 29.915) (width 0.2) (layer "F.Cu") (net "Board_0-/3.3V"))
 (segment (start 153 26.5) (end 150.33 26.5) (width 0.2) (layer "F.Cu") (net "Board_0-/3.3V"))
 (segment (start 150.48 26.891422) (end 150.48 26.608578) (width 0.2) (layer "F.Cu") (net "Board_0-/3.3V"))
 (segment (start 150.371422 26.5) (end 150.33 26.5) (width 0.2) (layer "F.Cu") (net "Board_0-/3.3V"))
 (segment (start 153.5 39.45) (end 153.25 39.7) (width 0.2) (layer "F.Cu") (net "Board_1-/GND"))
 (segment (start 150.48 39.308578) (end 150.48 39.591422) (width 0.2) (layer "F.Cu") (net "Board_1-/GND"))
 (segment (start 145.295 36.295) (end 147.466422 36.295) (width 0.2) (layer "F.Cu") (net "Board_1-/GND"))
 (segment (start 150.48 39.591422) (end 150.371422 39.7) (width 0.2) (layer "F.Cu") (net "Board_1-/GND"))
 (segment (start 153.25 39.7) (end 150.33 39.7) (width 0.2) (layer "F.Cu") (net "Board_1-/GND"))
 (segment (start 147.466422 36.295) (end 150.48 39.308578) (width 0.2) (layer "F.Cu") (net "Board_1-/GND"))
 (segment (start 150.371422 39.7) (end 150.33 39.7) (width 0.2) (layer "F.Cu") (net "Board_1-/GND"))
 (segment (start 145.295 38.835) (end 146.16 39.7) (width 0.2) (layer "F.Cu") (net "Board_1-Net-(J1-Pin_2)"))
 (segment (start 146.16 39.7) (end 148.93 39.7) (width 0.2) (layer "F.Cu") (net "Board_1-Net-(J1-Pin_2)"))
 (segment (start 146.17 40.5) (end 148.93 40.5) (width 0.2) (layer "F.Cu") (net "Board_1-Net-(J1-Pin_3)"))
 (segment (start 145.295 41.375) (end 146.17 40.5) (width 0.2) (layer "F.Cu") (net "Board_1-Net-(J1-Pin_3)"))
 (segment (start 150.371422 40.5) (end 150.33 40.5) (width 0.2) (layer "F.Cu") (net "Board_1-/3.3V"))
 (segment (start 150.48 40.891422) (end 150.48 40.608578) (width 0.2) (layer "F.Cu") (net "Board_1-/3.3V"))
 (segment (start 145.295 43.915) (end 147.456422 43.915) (width 0.2) (layer "F.Cu") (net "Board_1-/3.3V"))
 (segment (start 153.5 41) (end 153 40.5) (width 0.2) (layer "F.Cu") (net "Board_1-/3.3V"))
 (segment (start 147.456422 43.915) (end 150.48 40.891422) (width 0.2) (layer "F.Cu") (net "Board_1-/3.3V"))
 (segment (start 153 40.5) (end 150.33 40.5) (width 0.2) (layer "F.Cu") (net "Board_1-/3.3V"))
 (segment (start 150.48 40.608578) (end 150.371422 40.5) (width 0.2) (layer "F.Cu") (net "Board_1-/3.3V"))
 (segment (start 145.295 24.835) (end 146.16 25.7) (width 0.2) (layer "F.Cu") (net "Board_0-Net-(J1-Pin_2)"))
 (segment (start 146.16 25.7) (end 148.93 25.7) (width 0.2) (layer "F.Cu") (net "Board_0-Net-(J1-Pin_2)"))
 (segment (start 145.295 27.375) (end 146.17 26.5) (width 0.2) (layer "F.Cu") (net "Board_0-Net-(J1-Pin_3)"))
 (segment (start 146.17 26.5) (end 148.93 26.5) (width 0.2) (layer "F.Cu") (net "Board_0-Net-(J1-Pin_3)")))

